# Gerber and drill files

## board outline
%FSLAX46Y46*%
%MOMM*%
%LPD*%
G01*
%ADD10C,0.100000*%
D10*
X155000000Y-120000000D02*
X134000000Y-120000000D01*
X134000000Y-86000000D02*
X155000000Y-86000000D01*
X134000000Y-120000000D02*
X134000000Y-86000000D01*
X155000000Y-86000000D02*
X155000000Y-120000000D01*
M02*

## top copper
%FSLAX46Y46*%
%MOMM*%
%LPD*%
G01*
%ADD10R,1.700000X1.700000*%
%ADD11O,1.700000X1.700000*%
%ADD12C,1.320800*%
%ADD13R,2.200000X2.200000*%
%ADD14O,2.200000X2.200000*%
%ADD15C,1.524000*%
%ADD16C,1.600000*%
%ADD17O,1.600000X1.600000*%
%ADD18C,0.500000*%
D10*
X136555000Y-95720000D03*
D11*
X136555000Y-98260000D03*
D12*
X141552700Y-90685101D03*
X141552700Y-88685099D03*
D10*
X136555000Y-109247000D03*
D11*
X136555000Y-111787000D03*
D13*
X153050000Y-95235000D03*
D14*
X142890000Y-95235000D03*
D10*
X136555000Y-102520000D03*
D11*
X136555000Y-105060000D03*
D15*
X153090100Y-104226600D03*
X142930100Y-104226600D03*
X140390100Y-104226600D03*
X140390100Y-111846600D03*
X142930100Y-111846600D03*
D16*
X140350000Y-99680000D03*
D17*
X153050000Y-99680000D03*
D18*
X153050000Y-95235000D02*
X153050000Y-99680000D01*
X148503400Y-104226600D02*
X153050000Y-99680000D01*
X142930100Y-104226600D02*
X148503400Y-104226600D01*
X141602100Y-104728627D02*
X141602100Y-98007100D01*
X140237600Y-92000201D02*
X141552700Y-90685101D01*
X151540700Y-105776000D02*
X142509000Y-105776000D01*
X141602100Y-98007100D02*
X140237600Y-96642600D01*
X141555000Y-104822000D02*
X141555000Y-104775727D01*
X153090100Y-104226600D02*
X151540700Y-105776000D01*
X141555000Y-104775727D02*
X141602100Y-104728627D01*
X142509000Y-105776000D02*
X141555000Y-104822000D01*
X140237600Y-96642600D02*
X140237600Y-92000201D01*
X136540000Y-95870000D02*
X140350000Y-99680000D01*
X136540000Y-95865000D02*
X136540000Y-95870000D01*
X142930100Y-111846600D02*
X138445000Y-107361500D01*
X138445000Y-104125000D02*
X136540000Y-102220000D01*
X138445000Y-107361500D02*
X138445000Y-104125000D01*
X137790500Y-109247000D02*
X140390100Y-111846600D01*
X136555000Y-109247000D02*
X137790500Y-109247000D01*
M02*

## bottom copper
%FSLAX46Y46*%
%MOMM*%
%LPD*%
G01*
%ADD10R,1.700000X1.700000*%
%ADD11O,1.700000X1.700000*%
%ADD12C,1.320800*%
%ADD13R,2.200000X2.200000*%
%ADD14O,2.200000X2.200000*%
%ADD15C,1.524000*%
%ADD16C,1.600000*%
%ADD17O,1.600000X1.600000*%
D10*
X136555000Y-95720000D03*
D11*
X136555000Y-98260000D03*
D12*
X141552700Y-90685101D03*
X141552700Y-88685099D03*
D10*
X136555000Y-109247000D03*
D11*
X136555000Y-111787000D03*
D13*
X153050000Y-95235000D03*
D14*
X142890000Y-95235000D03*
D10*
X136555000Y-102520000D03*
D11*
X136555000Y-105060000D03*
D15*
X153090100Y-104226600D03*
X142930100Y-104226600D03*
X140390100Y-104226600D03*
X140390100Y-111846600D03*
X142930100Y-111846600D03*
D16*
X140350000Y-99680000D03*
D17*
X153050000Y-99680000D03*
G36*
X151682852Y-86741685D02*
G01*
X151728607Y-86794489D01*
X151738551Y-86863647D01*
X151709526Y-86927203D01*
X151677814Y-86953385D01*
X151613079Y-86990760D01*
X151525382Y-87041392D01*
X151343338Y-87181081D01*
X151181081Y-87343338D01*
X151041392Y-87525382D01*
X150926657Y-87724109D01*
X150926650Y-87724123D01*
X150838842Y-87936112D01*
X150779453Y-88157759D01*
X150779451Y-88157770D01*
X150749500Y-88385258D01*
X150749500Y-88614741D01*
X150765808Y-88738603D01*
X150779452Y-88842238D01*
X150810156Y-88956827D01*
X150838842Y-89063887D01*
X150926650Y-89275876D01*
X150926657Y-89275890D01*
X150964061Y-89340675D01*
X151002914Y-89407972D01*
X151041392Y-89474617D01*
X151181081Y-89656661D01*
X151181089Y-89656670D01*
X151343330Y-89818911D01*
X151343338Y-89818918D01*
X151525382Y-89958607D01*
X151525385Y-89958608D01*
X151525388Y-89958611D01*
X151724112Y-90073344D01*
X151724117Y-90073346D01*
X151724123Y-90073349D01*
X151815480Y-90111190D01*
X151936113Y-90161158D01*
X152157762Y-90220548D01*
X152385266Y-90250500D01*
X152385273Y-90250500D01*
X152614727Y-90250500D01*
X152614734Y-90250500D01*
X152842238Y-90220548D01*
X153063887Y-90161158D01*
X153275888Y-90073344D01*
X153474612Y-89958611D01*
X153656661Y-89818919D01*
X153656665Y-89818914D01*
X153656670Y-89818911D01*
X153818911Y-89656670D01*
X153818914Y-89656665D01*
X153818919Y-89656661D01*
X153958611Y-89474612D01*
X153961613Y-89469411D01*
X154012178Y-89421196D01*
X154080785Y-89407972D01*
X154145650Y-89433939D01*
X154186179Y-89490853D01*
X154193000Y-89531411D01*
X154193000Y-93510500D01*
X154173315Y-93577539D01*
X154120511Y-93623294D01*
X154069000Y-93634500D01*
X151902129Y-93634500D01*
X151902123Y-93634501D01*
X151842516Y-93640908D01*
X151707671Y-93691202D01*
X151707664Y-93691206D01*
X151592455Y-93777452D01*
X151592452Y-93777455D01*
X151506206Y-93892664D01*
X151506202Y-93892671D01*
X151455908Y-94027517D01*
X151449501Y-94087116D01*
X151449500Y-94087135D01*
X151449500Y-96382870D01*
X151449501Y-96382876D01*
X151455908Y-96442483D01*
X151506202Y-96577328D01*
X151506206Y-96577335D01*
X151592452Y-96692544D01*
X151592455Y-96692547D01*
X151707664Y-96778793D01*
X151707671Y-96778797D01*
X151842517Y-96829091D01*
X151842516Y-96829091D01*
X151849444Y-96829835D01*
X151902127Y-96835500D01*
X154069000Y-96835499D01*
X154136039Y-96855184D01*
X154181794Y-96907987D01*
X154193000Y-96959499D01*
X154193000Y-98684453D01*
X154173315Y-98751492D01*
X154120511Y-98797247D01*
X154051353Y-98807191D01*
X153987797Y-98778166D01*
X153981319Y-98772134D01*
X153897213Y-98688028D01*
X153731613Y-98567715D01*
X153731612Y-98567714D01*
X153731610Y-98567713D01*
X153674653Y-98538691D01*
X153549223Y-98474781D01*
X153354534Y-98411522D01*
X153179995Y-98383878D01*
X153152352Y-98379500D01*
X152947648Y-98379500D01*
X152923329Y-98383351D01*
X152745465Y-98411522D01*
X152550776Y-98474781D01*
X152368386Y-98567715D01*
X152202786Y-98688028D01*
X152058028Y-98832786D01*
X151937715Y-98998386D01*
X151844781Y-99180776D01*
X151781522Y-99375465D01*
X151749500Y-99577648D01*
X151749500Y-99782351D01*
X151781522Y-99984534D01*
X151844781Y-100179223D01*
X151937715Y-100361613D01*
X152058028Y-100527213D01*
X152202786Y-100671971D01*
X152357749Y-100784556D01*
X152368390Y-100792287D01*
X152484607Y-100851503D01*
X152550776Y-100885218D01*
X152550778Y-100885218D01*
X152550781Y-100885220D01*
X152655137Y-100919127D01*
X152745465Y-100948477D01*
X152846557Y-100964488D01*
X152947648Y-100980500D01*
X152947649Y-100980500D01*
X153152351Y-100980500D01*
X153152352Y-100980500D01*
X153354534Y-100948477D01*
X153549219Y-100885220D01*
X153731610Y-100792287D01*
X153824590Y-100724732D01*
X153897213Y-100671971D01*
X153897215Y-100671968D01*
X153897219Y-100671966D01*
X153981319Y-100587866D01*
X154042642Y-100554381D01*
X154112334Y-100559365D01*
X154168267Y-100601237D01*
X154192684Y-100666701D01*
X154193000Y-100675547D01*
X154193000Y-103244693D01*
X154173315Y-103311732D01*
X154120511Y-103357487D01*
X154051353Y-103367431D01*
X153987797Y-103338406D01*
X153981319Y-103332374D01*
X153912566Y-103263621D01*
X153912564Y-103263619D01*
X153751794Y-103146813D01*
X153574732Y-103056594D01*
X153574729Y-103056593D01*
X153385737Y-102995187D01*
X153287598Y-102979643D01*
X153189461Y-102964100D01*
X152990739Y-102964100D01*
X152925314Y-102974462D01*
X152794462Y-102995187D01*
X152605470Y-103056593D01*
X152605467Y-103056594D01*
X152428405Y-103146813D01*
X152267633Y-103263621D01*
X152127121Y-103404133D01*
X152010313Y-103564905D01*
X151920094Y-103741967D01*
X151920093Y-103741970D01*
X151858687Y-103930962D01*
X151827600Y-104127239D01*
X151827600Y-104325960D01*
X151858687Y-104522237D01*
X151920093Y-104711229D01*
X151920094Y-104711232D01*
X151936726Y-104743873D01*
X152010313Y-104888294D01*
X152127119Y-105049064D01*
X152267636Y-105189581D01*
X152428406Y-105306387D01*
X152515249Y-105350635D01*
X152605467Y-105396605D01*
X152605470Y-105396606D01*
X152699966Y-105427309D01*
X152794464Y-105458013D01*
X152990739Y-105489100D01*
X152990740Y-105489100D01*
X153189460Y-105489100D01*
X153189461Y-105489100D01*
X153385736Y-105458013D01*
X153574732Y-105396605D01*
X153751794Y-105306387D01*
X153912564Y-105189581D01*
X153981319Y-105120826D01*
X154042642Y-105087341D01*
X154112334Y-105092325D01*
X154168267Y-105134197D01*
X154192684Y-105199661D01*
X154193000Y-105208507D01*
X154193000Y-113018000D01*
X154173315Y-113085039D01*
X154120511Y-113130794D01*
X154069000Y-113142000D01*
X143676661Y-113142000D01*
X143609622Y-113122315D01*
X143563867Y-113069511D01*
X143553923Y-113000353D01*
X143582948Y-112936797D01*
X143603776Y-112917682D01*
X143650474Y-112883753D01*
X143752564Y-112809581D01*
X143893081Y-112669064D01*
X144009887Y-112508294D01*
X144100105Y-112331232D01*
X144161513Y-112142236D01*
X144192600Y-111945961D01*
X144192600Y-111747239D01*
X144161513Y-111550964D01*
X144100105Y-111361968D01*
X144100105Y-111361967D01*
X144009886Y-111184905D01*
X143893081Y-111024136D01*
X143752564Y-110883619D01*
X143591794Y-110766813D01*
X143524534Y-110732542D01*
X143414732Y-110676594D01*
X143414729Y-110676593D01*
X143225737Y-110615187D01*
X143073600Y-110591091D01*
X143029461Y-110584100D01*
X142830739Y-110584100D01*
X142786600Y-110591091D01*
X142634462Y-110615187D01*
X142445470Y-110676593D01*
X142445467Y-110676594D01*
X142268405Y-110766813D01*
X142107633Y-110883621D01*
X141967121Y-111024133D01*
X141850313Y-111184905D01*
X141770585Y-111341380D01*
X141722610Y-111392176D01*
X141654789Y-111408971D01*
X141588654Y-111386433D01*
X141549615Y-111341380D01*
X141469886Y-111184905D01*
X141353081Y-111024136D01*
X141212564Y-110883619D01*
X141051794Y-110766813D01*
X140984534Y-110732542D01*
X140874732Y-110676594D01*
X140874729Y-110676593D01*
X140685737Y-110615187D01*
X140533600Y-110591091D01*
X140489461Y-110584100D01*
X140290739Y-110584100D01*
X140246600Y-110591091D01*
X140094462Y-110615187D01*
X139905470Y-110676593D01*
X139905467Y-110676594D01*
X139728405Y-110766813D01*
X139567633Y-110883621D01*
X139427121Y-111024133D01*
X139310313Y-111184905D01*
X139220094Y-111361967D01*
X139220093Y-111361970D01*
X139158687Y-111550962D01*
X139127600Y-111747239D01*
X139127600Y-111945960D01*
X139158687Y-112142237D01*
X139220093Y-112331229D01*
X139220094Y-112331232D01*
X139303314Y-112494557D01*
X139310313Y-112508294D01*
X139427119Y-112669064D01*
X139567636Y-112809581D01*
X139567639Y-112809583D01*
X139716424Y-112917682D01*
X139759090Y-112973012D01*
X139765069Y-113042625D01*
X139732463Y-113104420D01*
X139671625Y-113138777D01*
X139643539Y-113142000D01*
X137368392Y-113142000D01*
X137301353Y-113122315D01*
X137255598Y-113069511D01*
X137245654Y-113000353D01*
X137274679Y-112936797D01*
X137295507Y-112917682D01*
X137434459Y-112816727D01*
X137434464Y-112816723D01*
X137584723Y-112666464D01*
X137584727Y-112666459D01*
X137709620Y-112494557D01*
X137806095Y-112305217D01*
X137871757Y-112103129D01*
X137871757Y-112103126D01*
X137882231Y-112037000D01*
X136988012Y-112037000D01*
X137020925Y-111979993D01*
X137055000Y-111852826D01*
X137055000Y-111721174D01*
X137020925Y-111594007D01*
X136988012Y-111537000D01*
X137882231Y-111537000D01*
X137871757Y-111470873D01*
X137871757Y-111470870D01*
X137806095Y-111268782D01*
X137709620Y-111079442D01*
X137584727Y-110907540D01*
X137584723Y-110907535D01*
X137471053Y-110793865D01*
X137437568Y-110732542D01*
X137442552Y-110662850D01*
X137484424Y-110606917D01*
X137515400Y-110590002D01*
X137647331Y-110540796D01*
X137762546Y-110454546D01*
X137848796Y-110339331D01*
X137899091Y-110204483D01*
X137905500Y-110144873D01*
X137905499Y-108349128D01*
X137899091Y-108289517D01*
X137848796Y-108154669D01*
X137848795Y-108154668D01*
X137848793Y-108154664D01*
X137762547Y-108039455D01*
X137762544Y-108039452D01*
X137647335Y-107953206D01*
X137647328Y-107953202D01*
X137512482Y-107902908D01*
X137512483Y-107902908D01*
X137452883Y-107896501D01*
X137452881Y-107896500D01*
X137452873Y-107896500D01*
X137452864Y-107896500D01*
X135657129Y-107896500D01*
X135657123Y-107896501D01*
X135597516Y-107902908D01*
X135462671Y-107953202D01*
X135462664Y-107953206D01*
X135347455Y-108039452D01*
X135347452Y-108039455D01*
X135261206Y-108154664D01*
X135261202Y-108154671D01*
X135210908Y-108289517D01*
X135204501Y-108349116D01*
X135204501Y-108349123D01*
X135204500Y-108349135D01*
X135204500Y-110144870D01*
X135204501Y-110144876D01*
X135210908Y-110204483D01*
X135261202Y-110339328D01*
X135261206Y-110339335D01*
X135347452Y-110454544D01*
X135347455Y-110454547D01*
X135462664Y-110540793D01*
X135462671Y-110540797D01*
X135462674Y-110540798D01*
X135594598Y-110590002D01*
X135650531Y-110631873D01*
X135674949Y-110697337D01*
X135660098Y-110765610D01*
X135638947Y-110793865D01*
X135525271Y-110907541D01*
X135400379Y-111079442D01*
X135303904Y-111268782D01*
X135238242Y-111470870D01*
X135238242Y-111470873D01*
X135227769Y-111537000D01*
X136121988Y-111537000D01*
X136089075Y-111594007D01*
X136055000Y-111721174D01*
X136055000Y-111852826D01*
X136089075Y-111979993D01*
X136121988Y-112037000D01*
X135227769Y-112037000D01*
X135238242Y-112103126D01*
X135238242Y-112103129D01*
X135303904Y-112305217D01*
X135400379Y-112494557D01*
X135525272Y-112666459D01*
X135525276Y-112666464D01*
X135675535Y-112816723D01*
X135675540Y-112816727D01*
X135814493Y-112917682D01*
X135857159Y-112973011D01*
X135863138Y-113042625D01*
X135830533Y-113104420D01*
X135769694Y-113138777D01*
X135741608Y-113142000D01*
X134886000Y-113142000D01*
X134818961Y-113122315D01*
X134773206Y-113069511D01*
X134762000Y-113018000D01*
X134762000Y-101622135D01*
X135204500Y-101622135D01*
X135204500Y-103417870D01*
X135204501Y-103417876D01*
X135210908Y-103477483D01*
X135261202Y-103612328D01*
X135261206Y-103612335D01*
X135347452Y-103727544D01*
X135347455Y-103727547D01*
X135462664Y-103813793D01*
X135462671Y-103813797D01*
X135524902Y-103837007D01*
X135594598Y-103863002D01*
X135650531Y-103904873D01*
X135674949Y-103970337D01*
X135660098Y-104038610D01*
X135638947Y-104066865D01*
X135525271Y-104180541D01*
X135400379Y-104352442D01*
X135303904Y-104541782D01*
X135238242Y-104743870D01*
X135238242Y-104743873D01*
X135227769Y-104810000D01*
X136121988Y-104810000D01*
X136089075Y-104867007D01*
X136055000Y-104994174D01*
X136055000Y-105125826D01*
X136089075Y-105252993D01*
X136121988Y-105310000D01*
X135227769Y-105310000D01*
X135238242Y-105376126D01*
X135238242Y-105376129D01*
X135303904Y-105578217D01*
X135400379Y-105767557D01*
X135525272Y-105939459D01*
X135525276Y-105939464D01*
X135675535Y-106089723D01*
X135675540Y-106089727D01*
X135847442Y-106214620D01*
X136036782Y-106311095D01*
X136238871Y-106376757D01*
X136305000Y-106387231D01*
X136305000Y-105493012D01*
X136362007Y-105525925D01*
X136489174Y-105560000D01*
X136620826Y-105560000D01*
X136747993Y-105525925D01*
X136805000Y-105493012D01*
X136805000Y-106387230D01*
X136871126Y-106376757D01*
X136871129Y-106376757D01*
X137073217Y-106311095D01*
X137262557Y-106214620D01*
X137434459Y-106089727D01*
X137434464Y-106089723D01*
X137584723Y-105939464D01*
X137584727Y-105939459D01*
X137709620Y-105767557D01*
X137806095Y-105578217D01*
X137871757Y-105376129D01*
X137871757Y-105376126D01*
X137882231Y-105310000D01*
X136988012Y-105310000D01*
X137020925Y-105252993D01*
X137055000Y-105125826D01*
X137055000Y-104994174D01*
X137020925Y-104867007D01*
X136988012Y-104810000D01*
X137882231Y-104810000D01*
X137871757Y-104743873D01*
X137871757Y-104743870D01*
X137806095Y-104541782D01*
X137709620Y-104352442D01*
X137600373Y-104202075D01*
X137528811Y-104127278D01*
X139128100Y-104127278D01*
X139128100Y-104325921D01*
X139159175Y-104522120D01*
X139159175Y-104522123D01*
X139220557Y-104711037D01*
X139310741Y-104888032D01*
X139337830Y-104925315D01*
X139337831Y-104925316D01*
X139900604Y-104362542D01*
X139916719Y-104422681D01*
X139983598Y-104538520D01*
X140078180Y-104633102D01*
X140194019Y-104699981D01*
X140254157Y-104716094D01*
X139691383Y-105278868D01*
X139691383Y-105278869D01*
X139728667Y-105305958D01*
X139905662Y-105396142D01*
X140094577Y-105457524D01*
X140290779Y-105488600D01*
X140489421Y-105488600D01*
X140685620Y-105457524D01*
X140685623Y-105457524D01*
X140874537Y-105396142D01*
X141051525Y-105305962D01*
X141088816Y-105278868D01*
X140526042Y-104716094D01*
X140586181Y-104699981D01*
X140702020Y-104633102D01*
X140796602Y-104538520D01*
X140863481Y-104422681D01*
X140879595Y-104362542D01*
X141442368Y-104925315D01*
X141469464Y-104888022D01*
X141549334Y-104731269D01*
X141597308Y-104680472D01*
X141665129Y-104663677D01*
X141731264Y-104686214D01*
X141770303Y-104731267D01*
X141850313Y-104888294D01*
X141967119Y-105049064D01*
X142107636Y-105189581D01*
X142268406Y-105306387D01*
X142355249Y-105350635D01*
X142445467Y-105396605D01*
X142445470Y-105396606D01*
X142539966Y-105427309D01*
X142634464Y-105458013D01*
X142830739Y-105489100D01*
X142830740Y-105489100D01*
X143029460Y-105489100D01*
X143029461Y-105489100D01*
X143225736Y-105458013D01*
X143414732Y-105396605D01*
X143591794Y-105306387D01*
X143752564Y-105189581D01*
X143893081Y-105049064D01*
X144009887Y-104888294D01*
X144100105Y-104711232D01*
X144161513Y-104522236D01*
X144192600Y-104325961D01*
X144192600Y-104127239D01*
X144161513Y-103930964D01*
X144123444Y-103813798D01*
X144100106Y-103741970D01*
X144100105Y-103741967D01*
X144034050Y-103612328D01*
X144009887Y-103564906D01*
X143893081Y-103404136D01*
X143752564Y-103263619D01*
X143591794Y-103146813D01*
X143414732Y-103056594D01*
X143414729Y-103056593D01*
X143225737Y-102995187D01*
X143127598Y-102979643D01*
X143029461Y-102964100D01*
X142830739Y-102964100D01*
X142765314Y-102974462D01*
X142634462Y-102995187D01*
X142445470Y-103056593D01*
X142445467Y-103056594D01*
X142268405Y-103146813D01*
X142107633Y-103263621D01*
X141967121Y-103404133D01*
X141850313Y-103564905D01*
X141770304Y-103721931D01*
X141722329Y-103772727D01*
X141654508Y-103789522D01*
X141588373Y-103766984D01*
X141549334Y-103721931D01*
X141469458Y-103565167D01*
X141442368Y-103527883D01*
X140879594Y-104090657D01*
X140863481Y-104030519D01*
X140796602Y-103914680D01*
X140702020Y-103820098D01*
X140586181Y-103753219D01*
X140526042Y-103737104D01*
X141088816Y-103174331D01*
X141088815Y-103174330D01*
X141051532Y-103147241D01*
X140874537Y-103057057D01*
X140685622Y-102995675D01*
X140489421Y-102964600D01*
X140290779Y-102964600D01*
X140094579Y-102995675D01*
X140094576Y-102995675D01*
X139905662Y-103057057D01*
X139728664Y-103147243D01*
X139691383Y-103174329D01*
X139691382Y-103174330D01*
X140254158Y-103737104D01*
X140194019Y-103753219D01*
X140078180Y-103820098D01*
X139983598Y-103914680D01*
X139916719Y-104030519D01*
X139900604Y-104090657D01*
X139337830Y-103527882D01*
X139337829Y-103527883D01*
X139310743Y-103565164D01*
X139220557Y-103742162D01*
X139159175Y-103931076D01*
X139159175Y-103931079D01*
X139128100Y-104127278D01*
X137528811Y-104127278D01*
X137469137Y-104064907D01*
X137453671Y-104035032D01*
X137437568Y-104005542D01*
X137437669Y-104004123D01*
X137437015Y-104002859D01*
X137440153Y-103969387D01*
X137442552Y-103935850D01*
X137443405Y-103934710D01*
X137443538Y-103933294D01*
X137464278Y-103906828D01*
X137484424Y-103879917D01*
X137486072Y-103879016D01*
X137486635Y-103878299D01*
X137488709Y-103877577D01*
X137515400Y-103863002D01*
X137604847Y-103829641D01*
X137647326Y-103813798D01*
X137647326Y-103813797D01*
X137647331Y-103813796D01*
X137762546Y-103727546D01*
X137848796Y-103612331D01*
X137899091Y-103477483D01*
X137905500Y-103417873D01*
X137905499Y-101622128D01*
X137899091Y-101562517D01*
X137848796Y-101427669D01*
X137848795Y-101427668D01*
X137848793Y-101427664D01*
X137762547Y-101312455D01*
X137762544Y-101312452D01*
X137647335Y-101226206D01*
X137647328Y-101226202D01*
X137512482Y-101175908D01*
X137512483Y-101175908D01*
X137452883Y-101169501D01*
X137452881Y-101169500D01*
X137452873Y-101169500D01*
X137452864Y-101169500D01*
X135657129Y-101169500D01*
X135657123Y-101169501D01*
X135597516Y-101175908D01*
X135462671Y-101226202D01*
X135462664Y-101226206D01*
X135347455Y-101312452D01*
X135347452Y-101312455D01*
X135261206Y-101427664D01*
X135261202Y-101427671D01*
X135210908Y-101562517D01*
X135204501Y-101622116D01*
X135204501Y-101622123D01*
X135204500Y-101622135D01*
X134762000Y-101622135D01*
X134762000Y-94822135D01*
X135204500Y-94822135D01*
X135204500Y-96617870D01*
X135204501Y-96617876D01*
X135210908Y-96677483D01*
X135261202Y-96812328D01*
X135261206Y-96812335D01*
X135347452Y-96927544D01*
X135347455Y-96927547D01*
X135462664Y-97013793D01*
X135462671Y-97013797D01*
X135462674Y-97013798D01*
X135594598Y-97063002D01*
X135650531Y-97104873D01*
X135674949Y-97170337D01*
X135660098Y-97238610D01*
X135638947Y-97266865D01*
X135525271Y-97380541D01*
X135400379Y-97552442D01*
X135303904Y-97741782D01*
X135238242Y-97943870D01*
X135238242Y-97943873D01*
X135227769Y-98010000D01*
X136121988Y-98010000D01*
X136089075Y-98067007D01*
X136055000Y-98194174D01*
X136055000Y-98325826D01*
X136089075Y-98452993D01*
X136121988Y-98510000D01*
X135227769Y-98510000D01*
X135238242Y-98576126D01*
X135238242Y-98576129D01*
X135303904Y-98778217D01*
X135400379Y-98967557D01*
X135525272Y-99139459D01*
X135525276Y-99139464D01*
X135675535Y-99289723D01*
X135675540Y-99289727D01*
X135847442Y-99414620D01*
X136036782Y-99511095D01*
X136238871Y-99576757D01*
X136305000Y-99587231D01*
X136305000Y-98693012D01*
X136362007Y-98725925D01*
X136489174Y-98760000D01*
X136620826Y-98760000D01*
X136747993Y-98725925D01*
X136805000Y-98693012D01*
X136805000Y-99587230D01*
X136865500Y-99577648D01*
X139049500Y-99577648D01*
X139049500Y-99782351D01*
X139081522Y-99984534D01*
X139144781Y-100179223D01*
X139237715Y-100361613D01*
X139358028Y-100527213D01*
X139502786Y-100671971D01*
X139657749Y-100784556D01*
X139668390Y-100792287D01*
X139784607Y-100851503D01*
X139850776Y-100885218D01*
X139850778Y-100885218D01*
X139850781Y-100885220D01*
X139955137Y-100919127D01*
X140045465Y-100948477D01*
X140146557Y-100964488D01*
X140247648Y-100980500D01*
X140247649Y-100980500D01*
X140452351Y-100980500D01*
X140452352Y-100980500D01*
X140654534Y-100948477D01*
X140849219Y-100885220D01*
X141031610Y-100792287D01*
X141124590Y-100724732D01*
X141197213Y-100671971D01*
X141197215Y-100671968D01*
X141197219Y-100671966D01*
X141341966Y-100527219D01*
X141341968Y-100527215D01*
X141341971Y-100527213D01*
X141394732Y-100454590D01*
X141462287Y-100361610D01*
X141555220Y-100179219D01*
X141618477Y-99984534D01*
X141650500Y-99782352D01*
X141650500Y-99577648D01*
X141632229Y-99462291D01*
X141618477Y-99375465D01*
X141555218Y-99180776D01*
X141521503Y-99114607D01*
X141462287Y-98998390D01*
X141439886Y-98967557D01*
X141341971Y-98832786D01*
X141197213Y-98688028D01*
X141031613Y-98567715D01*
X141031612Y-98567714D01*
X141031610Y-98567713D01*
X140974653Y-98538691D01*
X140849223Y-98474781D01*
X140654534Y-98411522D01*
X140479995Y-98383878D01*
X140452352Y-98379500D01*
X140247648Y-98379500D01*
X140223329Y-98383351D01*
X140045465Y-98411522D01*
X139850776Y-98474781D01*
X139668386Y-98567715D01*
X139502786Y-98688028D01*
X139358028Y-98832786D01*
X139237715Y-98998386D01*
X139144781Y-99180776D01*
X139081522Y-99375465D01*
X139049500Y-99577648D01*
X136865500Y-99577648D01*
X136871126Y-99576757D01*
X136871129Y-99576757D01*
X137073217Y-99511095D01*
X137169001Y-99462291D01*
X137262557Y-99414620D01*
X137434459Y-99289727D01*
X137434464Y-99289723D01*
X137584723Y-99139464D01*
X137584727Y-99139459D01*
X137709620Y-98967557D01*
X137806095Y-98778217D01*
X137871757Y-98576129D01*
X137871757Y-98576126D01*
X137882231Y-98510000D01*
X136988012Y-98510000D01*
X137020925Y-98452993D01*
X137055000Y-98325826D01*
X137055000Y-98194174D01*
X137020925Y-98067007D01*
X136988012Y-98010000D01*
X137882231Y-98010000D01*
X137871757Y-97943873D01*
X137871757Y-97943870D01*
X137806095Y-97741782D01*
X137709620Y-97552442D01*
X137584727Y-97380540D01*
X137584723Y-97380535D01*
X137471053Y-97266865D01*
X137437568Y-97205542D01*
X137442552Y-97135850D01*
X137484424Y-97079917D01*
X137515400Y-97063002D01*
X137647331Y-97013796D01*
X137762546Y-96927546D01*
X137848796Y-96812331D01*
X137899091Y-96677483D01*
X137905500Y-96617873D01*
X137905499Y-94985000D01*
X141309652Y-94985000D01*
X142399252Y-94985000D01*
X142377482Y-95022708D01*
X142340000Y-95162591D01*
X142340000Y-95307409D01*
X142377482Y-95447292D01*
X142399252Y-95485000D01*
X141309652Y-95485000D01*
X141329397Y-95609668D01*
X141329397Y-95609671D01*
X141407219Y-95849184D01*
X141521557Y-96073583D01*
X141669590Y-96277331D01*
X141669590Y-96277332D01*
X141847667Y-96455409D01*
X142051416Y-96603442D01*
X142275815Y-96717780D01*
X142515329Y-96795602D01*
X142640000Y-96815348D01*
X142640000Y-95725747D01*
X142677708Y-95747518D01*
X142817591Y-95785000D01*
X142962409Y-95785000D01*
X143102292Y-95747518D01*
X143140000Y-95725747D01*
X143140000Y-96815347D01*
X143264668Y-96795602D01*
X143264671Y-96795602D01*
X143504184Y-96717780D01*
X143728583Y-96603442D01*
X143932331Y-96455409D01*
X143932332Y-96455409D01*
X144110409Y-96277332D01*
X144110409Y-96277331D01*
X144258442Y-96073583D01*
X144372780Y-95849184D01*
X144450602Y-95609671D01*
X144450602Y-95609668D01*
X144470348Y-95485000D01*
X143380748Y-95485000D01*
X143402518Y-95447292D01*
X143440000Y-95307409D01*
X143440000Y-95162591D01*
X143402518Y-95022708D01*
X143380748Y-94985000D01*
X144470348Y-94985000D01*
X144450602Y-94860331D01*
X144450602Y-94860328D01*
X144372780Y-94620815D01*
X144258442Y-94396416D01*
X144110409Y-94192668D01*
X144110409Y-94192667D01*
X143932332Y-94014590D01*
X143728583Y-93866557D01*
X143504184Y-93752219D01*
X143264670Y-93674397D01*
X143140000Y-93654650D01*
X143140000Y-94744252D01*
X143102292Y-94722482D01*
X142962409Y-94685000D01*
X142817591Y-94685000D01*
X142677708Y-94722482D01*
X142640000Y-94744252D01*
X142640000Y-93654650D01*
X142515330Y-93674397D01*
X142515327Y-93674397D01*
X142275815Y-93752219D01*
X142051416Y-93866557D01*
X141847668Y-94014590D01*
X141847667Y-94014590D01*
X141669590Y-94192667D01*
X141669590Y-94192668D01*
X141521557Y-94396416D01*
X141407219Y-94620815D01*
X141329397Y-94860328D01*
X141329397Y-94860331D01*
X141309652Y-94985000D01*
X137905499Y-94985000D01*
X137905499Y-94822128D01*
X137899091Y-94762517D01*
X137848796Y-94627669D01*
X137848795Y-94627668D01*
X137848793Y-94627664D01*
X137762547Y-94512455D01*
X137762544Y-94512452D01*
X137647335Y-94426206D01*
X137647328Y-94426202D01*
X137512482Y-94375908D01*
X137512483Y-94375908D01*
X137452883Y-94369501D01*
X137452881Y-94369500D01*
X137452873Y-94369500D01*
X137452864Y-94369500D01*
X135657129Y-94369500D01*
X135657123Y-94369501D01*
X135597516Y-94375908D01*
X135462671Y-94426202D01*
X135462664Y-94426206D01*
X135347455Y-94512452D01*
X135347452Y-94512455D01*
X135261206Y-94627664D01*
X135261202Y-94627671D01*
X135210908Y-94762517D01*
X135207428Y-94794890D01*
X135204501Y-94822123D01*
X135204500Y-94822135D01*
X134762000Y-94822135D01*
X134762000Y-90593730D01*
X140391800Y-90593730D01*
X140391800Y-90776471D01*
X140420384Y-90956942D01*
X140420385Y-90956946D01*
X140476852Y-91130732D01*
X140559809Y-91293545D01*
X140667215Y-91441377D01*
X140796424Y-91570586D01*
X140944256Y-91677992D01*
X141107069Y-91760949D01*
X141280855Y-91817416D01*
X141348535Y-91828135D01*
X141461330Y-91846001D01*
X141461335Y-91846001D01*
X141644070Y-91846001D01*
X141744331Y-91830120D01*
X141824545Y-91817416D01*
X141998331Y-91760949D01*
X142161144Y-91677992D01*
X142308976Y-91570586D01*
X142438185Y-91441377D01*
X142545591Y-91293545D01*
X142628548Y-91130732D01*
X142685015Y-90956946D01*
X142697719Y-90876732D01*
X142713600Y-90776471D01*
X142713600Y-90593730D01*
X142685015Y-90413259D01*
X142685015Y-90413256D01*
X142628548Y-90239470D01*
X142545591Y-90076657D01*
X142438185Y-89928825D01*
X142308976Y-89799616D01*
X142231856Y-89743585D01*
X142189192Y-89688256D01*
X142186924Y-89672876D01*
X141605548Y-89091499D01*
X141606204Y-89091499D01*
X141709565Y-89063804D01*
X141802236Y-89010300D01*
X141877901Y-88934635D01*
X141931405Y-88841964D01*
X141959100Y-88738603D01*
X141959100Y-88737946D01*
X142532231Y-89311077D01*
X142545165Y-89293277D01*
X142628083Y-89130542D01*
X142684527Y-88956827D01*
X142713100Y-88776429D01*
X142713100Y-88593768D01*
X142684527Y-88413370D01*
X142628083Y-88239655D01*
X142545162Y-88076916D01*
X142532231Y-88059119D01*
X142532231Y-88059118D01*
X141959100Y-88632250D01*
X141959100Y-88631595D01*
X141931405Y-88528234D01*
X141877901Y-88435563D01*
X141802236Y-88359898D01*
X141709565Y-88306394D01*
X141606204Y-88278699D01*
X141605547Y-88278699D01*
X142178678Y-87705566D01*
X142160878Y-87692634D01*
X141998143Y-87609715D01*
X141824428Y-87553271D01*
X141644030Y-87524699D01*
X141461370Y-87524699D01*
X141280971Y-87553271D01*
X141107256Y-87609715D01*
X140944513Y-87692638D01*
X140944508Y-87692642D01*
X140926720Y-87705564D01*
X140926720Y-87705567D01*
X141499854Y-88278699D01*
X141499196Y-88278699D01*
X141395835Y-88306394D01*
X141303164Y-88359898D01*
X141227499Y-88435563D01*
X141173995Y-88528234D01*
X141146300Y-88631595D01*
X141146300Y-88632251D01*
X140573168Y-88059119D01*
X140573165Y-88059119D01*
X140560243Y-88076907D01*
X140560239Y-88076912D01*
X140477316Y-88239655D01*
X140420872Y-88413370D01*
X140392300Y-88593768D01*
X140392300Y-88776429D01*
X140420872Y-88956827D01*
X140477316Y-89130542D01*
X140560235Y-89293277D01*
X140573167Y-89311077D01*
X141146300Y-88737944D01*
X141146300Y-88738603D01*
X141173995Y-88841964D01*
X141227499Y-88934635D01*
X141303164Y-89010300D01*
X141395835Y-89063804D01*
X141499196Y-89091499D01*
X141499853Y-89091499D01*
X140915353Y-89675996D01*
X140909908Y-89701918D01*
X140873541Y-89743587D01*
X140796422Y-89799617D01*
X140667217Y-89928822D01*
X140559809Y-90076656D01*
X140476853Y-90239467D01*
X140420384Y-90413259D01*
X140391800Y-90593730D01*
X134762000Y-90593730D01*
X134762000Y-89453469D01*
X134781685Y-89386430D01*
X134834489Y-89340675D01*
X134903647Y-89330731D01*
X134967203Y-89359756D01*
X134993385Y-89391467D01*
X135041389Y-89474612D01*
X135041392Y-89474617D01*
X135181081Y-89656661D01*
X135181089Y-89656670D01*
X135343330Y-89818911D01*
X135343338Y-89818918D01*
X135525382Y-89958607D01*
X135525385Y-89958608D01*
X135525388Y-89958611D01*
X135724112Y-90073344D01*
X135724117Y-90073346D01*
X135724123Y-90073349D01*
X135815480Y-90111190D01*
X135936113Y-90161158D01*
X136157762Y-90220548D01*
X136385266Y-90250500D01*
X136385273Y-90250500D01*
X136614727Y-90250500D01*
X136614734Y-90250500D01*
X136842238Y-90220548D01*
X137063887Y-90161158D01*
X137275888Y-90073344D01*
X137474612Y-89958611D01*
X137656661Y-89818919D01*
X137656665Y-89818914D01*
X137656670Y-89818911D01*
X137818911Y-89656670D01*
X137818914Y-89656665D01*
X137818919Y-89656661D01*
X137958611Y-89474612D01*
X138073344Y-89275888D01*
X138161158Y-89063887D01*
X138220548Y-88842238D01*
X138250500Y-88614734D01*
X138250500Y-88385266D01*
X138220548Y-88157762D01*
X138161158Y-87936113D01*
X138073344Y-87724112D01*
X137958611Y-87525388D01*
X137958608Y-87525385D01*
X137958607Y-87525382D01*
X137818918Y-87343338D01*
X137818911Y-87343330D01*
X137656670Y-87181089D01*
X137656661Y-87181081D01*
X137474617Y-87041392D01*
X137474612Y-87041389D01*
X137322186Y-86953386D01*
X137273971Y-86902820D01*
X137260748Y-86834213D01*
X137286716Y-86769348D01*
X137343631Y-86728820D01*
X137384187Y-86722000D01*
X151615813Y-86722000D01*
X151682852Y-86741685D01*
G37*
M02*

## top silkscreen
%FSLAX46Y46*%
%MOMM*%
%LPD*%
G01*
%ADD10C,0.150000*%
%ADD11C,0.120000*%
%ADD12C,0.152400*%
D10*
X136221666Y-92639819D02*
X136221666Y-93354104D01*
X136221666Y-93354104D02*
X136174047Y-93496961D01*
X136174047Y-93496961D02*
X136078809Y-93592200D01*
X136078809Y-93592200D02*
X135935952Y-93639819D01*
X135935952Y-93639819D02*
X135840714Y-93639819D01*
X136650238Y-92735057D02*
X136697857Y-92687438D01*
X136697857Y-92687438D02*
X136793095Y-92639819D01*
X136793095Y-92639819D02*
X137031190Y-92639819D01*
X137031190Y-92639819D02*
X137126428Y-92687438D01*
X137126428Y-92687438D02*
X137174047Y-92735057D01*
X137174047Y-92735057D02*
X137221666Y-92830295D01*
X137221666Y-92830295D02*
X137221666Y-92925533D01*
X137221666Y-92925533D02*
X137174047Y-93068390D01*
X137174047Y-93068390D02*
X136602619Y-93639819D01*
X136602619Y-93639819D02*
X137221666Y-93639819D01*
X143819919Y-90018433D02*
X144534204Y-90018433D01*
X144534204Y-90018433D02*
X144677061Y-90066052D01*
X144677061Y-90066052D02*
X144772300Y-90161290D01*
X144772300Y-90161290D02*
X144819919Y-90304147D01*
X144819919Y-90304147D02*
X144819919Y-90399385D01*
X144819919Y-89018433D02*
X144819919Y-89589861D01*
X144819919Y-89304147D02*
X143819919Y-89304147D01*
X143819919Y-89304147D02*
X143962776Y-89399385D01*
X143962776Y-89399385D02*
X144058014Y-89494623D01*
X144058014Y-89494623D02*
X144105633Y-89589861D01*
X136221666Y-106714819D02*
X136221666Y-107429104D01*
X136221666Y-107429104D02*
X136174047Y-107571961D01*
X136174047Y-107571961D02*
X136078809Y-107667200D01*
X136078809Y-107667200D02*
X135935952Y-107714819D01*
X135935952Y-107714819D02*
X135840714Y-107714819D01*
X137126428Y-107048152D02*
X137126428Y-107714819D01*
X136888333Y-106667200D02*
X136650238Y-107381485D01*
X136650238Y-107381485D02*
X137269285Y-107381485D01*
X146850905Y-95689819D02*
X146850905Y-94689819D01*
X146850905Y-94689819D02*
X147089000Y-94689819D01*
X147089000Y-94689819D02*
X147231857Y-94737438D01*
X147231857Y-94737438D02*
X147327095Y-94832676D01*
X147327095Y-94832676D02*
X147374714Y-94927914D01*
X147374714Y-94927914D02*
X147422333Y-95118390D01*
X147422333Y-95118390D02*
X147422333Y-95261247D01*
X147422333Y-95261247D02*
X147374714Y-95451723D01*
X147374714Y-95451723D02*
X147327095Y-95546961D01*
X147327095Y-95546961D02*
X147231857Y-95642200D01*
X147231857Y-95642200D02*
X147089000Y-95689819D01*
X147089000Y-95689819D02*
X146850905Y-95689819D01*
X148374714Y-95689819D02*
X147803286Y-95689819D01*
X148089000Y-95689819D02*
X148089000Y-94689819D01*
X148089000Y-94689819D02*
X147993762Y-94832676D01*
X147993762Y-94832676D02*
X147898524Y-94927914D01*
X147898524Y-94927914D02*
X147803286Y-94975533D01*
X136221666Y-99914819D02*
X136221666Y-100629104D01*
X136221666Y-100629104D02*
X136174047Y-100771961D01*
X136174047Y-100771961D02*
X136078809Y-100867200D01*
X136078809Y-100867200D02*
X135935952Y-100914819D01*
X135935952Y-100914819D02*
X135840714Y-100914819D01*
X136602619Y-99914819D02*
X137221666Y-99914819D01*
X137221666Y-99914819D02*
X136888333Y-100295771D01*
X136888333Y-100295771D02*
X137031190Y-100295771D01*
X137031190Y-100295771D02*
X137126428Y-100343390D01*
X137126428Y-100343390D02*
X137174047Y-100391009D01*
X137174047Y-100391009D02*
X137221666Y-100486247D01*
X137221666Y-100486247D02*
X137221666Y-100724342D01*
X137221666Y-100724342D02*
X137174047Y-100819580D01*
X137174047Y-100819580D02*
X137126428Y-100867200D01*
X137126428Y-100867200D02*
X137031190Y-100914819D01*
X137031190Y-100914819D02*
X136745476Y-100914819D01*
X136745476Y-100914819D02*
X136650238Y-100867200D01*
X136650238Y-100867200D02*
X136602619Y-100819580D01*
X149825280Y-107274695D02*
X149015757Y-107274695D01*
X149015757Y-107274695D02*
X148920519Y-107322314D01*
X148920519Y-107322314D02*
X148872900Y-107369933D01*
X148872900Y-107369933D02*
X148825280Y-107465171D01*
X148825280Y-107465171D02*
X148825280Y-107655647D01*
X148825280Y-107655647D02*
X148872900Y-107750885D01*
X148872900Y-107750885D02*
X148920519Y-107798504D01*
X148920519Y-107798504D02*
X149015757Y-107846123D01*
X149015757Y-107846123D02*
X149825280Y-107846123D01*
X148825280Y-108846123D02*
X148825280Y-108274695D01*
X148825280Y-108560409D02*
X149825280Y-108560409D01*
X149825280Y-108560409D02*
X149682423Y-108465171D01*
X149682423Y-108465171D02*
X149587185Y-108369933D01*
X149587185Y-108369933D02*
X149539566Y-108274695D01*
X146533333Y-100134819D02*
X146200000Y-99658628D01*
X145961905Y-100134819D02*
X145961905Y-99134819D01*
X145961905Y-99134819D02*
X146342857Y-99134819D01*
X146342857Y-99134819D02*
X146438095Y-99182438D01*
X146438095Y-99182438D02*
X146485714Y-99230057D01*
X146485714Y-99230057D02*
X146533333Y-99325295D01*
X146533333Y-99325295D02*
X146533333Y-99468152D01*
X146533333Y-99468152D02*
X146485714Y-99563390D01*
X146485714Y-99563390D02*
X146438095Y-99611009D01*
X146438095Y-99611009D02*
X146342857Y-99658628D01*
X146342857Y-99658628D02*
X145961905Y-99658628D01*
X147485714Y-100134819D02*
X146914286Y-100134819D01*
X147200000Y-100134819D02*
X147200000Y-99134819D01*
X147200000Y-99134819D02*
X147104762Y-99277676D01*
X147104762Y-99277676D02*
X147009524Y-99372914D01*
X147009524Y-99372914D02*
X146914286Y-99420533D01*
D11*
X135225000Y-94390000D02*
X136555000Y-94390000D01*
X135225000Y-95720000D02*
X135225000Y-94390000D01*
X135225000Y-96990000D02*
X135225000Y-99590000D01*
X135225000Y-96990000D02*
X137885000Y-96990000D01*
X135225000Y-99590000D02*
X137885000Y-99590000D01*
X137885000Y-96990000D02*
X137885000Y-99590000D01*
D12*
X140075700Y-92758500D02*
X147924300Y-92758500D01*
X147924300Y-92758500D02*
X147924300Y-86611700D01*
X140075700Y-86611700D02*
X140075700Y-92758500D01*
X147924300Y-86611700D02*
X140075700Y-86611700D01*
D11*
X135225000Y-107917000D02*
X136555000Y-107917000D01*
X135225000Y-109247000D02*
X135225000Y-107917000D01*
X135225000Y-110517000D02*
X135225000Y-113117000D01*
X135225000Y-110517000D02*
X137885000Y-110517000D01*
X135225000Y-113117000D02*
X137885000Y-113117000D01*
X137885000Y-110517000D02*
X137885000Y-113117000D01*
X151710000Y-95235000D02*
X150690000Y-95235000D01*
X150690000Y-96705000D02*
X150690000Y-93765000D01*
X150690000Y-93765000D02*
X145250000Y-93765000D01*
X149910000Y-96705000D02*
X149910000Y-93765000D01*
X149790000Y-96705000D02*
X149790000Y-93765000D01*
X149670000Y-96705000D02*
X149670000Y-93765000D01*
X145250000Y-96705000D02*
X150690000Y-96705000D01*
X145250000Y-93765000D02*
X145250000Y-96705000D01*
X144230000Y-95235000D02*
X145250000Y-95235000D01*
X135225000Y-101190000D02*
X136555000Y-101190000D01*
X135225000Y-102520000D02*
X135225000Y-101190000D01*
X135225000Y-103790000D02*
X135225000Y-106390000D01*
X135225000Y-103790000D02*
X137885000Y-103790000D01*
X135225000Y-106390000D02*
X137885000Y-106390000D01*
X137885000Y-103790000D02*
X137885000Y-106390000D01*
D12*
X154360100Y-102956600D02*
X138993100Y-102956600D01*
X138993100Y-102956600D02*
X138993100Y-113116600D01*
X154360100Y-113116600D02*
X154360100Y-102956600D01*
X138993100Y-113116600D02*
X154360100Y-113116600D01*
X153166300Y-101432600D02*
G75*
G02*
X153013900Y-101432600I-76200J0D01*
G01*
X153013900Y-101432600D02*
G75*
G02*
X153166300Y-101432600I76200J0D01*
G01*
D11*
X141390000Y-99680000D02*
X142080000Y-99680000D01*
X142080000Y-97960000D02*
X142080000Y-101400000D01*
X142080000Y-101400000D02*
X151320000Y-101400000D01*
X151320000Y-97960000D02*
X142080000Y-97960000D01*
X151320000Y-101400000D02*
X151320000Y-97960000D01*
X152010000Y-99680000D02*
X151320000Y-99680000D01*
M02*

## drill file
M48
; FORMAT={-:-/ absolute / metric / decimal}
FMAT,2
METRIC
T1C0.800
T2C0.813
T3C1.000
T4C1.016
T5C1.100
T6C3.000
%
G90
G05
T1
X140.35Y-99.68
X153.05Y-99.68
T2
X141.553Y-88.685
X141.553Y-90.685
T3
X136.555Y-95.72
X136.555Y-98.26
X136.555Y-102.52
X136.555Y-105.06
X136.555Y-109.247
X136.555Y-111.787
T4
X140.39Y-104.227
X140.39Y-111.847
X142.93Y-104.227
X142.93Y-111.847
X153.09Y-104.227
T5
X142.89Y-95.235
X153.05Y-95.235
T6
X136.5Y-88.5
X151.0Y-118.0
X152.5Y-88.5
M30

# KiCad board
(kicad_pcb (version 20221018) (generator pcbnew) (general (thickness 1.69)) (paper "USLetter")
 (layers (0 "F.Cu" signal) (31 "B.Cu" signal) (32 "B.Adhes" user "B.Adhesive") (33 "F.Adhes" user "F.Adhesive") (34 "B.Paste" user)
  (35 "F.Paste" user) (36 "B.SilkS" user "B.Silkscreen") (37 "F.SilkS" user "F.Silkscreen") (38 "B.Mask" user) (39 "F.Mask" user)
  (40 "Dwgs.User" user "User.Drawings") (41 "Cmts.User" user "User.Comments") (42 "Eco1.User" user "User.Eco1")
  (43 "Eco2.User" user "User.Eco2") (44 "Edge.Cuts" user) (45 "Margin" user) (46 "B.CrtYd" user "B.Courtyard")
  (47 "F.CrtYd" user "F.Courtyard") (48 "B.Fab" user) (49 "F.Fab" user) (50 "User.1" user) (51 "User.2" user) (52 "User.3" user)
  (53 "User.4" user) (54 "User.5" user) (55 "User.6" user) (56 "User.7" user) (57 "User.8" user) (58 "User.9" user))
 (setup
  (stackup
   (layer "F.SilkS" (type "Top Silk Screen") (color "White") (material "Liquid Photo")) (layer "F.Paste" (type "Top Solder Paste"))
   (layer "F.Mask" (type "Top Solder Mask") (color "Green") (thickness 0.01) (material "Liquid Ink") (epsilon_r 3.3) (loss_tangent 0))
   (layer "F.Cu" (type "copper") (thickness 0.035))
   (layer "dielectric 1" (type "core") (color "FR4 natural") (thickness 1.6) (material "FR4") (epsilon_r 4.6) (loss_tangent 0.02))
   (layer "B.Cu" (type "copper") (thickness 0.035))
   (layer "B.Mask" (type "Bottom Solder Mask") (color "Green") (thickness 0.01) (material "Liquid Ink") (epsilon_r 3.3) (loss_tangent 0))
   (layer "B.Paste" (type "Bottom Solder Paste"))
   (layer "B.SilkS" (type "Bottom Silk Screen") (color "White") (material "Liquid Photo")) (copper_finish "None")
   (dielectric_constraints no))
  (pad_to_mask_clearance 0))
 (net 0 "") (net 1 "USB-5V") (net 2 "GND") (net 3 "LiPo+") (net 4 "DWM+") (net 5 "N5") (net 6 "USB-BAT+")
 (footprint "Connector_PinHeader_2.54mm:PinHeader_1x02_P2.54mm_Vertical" (layer "F.Cu") (at 136.555 95.72)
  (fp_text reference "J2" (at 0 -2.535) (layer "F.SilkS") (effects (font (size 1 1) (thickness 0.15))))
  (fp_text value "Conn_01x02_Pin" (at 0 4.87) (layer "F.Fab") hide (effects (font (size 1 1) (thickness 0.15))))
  (fp_line (start -1.33 -1.33) (end 0 -1.33) (stroke (width 0.12) (type solid)) (layer "F.SilkS"))
  (fp_line (start -1.33 0) (end -1.33 -1.33) (stroke (width 0.12) (type solid)) (layer "F.SilkS"))
  (fp_line (start -1.33 1.27) (end -1.33 3.87) (stroke (width 0.12) (type solid)) (layer "F.SilkS"))
  (fp_line (start -1.33 1.27) (end 1.33 1.27) (stroke (width 0.12) (type solid)) (layer "F.SilkS"))
  (fp_line (start -1.33 3.87) (end 1.33 3.87) (stroke (width 0.12) (type solid)) (layer "F.SilkS"))
  (fp_line (start 1.33 1.27) (end 1.33 3.87) (stroke (width 0.12) (type solid)) (layer "F.SilkS"))
  (pad "1" thru_hole rect (at 0 0) (size 1.7 1.7) (drill 1) (layers "*.Cu" "*.Mask") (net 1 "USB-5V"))
  (pad "2" thru_hole oval (at 0 2.54) (size 1.7 1.7) (drill 1) (layers "*.Cu" "*.Mask") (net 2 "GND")))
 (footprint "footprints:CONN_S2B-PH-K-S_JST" (layer "F.Cu") (at 141.5527 90.6851 90)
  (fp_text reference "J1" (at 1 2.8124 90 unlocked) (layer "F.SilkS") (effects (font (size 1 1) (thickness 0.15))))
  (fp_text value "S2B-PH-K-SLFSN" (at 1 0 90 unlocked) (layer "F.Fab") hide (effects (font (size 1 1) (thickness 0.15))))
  (fp_line (start -2.0734 -1.477) (end -2.0734 6.3716) (stroke (width 0.1524) (type solid)) (layer "F.SilkS"))
  (fp_line (start -2.0734 6.3716) (end 4.0734 6.3716) (stroke (width 0.1524) (type solid)) (layer "F.SilkS"))
  (fp_line (start 4.0734 -1.477) (end -2.0734 -1.477) (stroke (width 0.1524) (type solid)) (layer "F.SilkS"))
  (fp_line (start 4.0734 6.3716) (end 4.0734 -1.477) (stroke (width 0.1524) (type solid)) (layer "F.SilkS"))
  (pad "1" thru_hole circle (at -0.000001 0 90) (size 1.3208 1.3208) (drill 0.8128) (layers "*.Cu" "*.Mask") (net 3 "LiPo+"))
  (pad "2" thru_hole circle (at 2.000001 0 90) (size 1.3208 1.3208) (drill 0.8128) (layers "*.Cu" "*.Mask") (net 2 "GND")))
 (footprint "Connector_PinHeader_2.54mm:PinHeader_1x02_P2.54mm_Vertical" (layer "F.Cu") (at 136.555 109.247)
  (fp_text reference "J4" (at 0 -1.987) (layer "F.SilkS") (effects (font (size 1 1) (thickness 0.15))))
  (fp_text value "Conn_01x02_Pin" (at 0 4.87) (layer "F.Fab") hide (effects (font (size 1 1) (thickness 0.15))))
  (fp_line (start -1.33 -1.33) (end 0 -1.33) (stroke (width 0.12) (type solid)) (layer "F.SilkS"))
  (fp_line (start -1.33 0) (end -1.33 -1.33) (stroke (width 0.12) (type solid)) (layer "F.SilkS"))
  (fp_line (start -1.33 1.27) (end -1.33 3.87) (stroke (width 0.12) (type solid)) (layer "F.SilkS"))
  (fp_line (start -1.33 1.27) (end 1.33 1.27) (stroke (width 0.12) (type solid)) (layer "F.SilkS"))
  (fp_line (start -1.33 3.87) (end 1.33 3.87) (stroke (width 0.12) (type solid)) (layer "F.SilkS"))
  (fp_line (start 1.33 1.27) (end 1.33 3.87) (stroke (width 0.12) (type solid)) (layer "F.SilkS"))
  (pad "1" thru_hole rect (at 0 0) (size 1.7 1.7) (drill 1) (layers "*.Cu" "*.Mask") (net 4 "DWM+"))
  (pad "2" thru_hole oval (at 0 2.54) (size 1.7 1.7) (drill 1) (layers "*.Cu" "*.Mask") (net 2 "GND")))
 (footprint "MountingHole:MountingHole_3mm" (layer "F.Cu") (at 152.5 88.5)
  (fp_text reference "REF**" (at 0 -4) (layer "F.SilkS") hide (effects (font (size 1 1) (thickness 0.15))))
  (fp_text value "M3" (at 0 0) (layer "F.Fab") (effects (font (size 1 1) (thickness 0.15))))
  (pad "" np_thru_hole circle (at 0 0) (size 3 3) (drill 3) (layers "F&B.Cu" "*.Mask")))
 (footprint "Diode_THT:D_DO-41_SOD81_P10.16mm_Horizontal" (layer "F.Cu") (at 153.05 95.235 180)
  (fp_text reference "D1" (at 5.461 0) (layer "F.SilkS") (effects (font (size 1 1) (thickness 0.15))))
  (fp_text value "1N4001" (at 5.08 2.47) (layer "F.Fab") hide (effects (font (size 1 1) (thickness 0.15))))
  (fp_line (start 1.34 0) (end 2.36 0) (stroke (width 0.12) (type solid)) (layer "F.SilkS"))
  (fp_line (start 2.36 -1.47) (end 2.36 1.47) (stroke (width 0.12) (type solid)) (layer "F.SilkS"))
  (fp_line (start 2.36 1.47) (end 7.8 1.47) (stroke (width 0.12) (type solid)) (layer "F.SilkS"))
  (fp_line (start 3.14 -1.47) (end 3.14 1.47) (stroke (width 0.12) (type solid)) (layer "F.SilkS"))
  (fp_line (start 3.26 -1.47) (end 3.26 1.47) (stroke (width 0.12) (type solid)) (layer "F.SilkS"))
  (fp_line (start 3.38 -1.47) (end 3.38 1.47) (stroke (width 0.12) (type solid)) (layer "F.SilkS"))
  (fp_line (start 7.8 -1.47) (end 2.36 -1.47) (stroke (width 0.12) (type solid)) (layer "F.SilkS"))
  (fp_line (start 7.8 1.47) (end 7.8 -1.47) (stroke (width 0.12) (type solid)) (layer "F.SilkS"))
  (fp_line (start 8.82 0) (end 7.8 0) (stroke (width 0.12) (type solid)) (layer "F.SilkS"))
  (pad "1" thru_hole rect (at 0 0 180) (size 2.2 2.2) (drill 1.1) (layers "*.Cu" "*.Mask") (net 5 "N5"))
  (pad "2" thru_hole oval (at 10.16 0 180) (size 2.2 2.2) (drill 1.1) (layers "*.Cu" "*.Mask") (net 2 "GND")))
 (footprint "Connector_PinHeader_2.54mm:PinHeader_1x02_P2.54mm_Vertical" (layer "F.Cu") (at 136.555 102.52)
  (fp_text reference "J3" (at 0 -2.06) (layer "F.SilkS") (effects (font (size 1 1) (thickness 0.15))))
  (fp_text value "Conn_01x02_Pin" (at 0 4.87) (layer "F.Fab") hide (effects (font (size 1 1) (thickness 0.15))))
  (fp_line (start -1.33 -1.33) (end 0 -1.33) (stroke (width 0.12) (type solid)) (layer "F.SilkS"))
  (fp_line (start -1.33 0) (end -1.33 -1.33) (stroke (width 0.12) (type solid)) (layer "F.SilkS"))
  (fp_line (start -1.33 1.27) (end -1.33 3.87) (stroke (width 0.12) (type solid)) (layer "F.SilkS"))
  (fp_line (start -1.33 1.27) (end 1.33 1.27) (stroke (width 0.12) (type solid)) (layer "F.SilkS"))
  (fp_line (start -1.33 3.87) (end 1.33 3.87) (stroke (width 0.12) (type solid)) (layer "F.SilkS"))
  (fp_line (start 1.33 1.27) (end 1.33 3.87) (stroke (width 0.12) (type solid)) (layer "F.SilkS"))
  (pad "1" thru_hole rect (at 0 0) (size 1.7 1.7) (drill 1) (layers "*.Cu" "*.Mask") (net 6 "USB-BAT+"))
  (pad "2" thru_hole oval (at 0 2.54) (size 1.7 1.7) (drill 1) (layers "*.Cu" "*.Mask") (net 2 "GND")))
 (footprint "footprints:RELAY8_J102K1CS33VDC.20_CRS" (layer "F.Cu") (at 158.1701 104.2266 -90)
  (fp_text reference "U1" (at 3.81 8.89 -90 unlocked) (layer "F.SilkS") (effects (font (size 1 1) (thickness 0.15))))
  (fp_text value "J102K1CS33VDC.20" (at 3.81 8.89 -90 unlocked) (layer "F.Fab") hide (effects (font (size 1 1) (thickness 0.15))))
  (fp_line (start -1.27 3.81) (end -1.27 19.177) (stroke (width 0.1524) (type solid)) (layer "F.SilkS"))
  (fp_line (start -1.27 19.177) (end 8.89 19.177) (stroke (width 0.1524) (type solid)) (layer "F.SilkS"))
  (fp_line (start 8.89 3.81) (end -1.27 3.81) (stroke (width 0.1524) (type solid)) (layer "F.SilkS"))
  (fp_line (start 8.89 19.177) (end 8.89 3.81) (stroke (width 0.1524) (type solid)) (layer "F.SilkS"))
  (fp_circle (center -2.794 5.08) (end -2.7178 5.08) (stroke (width 0.1524) (type solid)) (fill none) (layer "F.SilkS"))
  (pad "1" thru_hole circle (at 0 5.08 270) (size 1.524 1.524) (drill 1.016) (layers "*.Cu" "*.Mask") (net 3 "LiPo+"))
  (pad "3" thru_hole circle (at 0 15.24 270) (size 1.524 1.524) (drill 1.016) (layers "*.Cu" "*.Mask") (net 5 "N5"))
  (pad "4" thru_hole circle (at 0 17.78 270) (size 1.524 1.524) (drill 1.016) (layers "*.Cu" "*.Mask") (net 2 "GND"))
  (pad "5" thru_hole circle (at 7.62 17.78 270) (size 1.524 1.524) (drill 1.016) (layers "*.Cu" "*.Mask") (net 4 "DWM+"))
  (pad "6" thru_hole circle (at 7.62 15.24 270) (size 1.524 1.524) (drill 1.016) (layers "*.Cu" "*.Mask") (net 6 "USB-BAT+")))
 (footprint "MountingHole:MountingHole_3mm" (layer "F.Cu") (at 151 118)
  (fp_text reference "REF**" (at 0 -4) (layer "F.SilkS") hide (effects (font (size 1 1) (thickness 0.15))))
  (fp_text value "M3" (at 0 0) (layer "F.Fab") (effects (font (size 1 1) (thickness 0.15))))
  (pad "" np_thru_hole circle (at 0 0) (size 3 3) (drill 3) (layers "*.Cu" "*.Mask")))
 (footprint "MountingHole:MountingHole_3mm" (layer "F.Cu") (at 136.5 88.5)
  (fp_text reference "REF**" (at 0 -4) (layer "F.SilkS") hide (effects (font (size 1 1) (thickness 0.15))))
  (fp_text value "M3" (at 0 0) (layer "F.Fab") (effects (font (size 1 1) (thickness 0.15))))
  (pad "" np_thru_hole circle (at 0 0) (size 3 3) (drill 3) (layers "F&B.Cu" "*.Mask")))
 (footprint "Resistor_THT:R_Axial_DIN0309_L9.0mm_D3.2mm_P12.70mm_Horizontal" (layer "F.Cu") (at 140.35 99.68)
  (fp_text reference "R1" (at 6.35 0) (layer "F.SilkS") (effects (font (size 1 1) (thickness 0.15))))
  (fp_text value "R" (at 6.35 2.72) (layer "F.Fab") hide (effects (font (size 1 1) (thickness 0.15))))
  (fp_line (start 1.04 0) (end 1.73 0) (stroke (width 0.12) (type solid)) (layer "F.SilkS"))
  (fp_line (start 1.73 -1.72) (end 1.73 1.72) (stroke (width 0.12) (type solid)) (layer "F.SilkS"))
  (fp_line (start 1.73 1.72) (end 10.97 1.72) (stroke (width 0.12) (type solid)) (layer "F.SilkS"))
  (fp_line (start 10.97 -1.72) (end 1.73 -1.72) (stroke (width 0.12) (type solid)) (layer "F.SilkS"))
  (fp_line (start 10.97 1.72) (end 10.97 -1.72) (stroke (width 0.12) (type solid)) (layer "F.SilkS"))
  (fp_line (start 11.66 0) (end 10.97 0) (stroke (width 0.12) (type solid)) (layer "F.SilkS"))
  (pad "1" thru_hole circle (at 0 0) (size 1.6 1.6) (drill 0.8) (layers "*.Cu" "*.Mask") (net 1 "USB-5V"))
  (pad "2" thru_hole oval (at 12.7 0) (size 1.6 1.6) (drill 0.8) (layers "*.Cu" "*.Mask") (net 5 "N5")))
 (gr_line (start 155 120) (end 134 120) (stroke (width 0.1) (type default)) (layer "Edge.Cuts"))
 (gr_line (start 134 86) (end 155 86) (stroke (width 0.1) (type default)) (layer "Edge.Cuts"))
 (gr_line (start 134 120) (end 134 86) (stroke (width 0.1) (type default)) (layer "Edge.Cuts"))
 (gr_line (start 155 86) (end 155 120) (stroke (width 0.1) (type default)) (layer "Edge.Cuts"))
 (segment (start 153.05 95.235) (end 153.05 99.68) (width 0.5) (layer "F.Cu") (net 5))
 (segment (start 148.5034 104.2266) (end 153.05 99.68) (width 0.5) (layer "F.Cu") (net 5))
 (segment (start 142.9301 104.2266) (end 148.5034 104.2266) (width 0.5) (layer "F.Cu") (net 5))
 (segment (start 141.6021 104.728627) (end 141.6021 98.0071) (width 0.5) (layer "F.Cu") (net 3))
 (segment (start 140.2376 92.000201) (end 141.5527 90.685101) (width 0.5) (layer "F.Cu") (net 3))
 (segment (start 151.5407 105.776) (end 142.509 105.776) (width 0.5) (layer "F.Cu") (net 3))
 (segment (start 141.6021 98.0071) (end 140.2376 96.6426) (width 0.5) (layer "F.Cu") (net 3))
 (segment (start 141.555 104.822) (end 141.555 104.775727) (width 0.5) (layer "F.Cu") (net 3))
 (segment (start 153.0901 104.2266) (end 151.5407 105.776) (width 0.5) (layer "F.Cu") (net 3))
 (segment (start 141.555 104.775727) (end 141.6021 104.728627) (width 0.5) (layer "F.Cu") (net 3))
 (segment (start 142.509 105.776) (end 141.555 104.822) (width 0.5) (layer "F.Cu") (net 3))
 (segment (start 140.2376 96.6426) (end 140.2376 92.000201) (width 0.5) (layer "F.Cu") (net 3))
 (segment (start 136.54 95.87) (end 140.35 99.68) (width 0.5) (layer "F.Cu") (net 1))
 (segment (start 136.54 95.865) (end 136.54 95.87) (width 0.5) (layer "F.Cu") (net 1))
 (segment (start 142.9301 111.8466) (end 138.445 107.3615) (width 0.5) (layer "F.Cu") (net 6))
 (segment (start 138.445 104.125) (end 136.54 102.22) (width 0.5) (layer "F.Cu") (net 6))
 (segment (start 138.445 107.3615) (end 138.445 104.125) (width 0.5) (layer "F.Cu") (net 6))
 (segment (start 137.7905 109.247) (end 140.3901 111.8466) (width 0.5) (layer "F.Cu") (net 4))
 (segment (start 136.555 109.247) (end 137.7905 109.247) (width 0.5) (layer "F.Cu") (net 4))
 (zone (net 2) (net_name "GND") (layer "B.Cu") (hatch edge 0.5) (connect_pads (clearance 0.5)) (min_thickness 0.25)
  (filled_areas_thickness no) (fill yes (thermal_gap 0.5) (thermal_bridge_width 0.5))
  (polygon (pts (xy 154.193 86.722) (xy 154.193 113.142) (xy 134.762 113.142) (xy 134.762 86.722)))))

